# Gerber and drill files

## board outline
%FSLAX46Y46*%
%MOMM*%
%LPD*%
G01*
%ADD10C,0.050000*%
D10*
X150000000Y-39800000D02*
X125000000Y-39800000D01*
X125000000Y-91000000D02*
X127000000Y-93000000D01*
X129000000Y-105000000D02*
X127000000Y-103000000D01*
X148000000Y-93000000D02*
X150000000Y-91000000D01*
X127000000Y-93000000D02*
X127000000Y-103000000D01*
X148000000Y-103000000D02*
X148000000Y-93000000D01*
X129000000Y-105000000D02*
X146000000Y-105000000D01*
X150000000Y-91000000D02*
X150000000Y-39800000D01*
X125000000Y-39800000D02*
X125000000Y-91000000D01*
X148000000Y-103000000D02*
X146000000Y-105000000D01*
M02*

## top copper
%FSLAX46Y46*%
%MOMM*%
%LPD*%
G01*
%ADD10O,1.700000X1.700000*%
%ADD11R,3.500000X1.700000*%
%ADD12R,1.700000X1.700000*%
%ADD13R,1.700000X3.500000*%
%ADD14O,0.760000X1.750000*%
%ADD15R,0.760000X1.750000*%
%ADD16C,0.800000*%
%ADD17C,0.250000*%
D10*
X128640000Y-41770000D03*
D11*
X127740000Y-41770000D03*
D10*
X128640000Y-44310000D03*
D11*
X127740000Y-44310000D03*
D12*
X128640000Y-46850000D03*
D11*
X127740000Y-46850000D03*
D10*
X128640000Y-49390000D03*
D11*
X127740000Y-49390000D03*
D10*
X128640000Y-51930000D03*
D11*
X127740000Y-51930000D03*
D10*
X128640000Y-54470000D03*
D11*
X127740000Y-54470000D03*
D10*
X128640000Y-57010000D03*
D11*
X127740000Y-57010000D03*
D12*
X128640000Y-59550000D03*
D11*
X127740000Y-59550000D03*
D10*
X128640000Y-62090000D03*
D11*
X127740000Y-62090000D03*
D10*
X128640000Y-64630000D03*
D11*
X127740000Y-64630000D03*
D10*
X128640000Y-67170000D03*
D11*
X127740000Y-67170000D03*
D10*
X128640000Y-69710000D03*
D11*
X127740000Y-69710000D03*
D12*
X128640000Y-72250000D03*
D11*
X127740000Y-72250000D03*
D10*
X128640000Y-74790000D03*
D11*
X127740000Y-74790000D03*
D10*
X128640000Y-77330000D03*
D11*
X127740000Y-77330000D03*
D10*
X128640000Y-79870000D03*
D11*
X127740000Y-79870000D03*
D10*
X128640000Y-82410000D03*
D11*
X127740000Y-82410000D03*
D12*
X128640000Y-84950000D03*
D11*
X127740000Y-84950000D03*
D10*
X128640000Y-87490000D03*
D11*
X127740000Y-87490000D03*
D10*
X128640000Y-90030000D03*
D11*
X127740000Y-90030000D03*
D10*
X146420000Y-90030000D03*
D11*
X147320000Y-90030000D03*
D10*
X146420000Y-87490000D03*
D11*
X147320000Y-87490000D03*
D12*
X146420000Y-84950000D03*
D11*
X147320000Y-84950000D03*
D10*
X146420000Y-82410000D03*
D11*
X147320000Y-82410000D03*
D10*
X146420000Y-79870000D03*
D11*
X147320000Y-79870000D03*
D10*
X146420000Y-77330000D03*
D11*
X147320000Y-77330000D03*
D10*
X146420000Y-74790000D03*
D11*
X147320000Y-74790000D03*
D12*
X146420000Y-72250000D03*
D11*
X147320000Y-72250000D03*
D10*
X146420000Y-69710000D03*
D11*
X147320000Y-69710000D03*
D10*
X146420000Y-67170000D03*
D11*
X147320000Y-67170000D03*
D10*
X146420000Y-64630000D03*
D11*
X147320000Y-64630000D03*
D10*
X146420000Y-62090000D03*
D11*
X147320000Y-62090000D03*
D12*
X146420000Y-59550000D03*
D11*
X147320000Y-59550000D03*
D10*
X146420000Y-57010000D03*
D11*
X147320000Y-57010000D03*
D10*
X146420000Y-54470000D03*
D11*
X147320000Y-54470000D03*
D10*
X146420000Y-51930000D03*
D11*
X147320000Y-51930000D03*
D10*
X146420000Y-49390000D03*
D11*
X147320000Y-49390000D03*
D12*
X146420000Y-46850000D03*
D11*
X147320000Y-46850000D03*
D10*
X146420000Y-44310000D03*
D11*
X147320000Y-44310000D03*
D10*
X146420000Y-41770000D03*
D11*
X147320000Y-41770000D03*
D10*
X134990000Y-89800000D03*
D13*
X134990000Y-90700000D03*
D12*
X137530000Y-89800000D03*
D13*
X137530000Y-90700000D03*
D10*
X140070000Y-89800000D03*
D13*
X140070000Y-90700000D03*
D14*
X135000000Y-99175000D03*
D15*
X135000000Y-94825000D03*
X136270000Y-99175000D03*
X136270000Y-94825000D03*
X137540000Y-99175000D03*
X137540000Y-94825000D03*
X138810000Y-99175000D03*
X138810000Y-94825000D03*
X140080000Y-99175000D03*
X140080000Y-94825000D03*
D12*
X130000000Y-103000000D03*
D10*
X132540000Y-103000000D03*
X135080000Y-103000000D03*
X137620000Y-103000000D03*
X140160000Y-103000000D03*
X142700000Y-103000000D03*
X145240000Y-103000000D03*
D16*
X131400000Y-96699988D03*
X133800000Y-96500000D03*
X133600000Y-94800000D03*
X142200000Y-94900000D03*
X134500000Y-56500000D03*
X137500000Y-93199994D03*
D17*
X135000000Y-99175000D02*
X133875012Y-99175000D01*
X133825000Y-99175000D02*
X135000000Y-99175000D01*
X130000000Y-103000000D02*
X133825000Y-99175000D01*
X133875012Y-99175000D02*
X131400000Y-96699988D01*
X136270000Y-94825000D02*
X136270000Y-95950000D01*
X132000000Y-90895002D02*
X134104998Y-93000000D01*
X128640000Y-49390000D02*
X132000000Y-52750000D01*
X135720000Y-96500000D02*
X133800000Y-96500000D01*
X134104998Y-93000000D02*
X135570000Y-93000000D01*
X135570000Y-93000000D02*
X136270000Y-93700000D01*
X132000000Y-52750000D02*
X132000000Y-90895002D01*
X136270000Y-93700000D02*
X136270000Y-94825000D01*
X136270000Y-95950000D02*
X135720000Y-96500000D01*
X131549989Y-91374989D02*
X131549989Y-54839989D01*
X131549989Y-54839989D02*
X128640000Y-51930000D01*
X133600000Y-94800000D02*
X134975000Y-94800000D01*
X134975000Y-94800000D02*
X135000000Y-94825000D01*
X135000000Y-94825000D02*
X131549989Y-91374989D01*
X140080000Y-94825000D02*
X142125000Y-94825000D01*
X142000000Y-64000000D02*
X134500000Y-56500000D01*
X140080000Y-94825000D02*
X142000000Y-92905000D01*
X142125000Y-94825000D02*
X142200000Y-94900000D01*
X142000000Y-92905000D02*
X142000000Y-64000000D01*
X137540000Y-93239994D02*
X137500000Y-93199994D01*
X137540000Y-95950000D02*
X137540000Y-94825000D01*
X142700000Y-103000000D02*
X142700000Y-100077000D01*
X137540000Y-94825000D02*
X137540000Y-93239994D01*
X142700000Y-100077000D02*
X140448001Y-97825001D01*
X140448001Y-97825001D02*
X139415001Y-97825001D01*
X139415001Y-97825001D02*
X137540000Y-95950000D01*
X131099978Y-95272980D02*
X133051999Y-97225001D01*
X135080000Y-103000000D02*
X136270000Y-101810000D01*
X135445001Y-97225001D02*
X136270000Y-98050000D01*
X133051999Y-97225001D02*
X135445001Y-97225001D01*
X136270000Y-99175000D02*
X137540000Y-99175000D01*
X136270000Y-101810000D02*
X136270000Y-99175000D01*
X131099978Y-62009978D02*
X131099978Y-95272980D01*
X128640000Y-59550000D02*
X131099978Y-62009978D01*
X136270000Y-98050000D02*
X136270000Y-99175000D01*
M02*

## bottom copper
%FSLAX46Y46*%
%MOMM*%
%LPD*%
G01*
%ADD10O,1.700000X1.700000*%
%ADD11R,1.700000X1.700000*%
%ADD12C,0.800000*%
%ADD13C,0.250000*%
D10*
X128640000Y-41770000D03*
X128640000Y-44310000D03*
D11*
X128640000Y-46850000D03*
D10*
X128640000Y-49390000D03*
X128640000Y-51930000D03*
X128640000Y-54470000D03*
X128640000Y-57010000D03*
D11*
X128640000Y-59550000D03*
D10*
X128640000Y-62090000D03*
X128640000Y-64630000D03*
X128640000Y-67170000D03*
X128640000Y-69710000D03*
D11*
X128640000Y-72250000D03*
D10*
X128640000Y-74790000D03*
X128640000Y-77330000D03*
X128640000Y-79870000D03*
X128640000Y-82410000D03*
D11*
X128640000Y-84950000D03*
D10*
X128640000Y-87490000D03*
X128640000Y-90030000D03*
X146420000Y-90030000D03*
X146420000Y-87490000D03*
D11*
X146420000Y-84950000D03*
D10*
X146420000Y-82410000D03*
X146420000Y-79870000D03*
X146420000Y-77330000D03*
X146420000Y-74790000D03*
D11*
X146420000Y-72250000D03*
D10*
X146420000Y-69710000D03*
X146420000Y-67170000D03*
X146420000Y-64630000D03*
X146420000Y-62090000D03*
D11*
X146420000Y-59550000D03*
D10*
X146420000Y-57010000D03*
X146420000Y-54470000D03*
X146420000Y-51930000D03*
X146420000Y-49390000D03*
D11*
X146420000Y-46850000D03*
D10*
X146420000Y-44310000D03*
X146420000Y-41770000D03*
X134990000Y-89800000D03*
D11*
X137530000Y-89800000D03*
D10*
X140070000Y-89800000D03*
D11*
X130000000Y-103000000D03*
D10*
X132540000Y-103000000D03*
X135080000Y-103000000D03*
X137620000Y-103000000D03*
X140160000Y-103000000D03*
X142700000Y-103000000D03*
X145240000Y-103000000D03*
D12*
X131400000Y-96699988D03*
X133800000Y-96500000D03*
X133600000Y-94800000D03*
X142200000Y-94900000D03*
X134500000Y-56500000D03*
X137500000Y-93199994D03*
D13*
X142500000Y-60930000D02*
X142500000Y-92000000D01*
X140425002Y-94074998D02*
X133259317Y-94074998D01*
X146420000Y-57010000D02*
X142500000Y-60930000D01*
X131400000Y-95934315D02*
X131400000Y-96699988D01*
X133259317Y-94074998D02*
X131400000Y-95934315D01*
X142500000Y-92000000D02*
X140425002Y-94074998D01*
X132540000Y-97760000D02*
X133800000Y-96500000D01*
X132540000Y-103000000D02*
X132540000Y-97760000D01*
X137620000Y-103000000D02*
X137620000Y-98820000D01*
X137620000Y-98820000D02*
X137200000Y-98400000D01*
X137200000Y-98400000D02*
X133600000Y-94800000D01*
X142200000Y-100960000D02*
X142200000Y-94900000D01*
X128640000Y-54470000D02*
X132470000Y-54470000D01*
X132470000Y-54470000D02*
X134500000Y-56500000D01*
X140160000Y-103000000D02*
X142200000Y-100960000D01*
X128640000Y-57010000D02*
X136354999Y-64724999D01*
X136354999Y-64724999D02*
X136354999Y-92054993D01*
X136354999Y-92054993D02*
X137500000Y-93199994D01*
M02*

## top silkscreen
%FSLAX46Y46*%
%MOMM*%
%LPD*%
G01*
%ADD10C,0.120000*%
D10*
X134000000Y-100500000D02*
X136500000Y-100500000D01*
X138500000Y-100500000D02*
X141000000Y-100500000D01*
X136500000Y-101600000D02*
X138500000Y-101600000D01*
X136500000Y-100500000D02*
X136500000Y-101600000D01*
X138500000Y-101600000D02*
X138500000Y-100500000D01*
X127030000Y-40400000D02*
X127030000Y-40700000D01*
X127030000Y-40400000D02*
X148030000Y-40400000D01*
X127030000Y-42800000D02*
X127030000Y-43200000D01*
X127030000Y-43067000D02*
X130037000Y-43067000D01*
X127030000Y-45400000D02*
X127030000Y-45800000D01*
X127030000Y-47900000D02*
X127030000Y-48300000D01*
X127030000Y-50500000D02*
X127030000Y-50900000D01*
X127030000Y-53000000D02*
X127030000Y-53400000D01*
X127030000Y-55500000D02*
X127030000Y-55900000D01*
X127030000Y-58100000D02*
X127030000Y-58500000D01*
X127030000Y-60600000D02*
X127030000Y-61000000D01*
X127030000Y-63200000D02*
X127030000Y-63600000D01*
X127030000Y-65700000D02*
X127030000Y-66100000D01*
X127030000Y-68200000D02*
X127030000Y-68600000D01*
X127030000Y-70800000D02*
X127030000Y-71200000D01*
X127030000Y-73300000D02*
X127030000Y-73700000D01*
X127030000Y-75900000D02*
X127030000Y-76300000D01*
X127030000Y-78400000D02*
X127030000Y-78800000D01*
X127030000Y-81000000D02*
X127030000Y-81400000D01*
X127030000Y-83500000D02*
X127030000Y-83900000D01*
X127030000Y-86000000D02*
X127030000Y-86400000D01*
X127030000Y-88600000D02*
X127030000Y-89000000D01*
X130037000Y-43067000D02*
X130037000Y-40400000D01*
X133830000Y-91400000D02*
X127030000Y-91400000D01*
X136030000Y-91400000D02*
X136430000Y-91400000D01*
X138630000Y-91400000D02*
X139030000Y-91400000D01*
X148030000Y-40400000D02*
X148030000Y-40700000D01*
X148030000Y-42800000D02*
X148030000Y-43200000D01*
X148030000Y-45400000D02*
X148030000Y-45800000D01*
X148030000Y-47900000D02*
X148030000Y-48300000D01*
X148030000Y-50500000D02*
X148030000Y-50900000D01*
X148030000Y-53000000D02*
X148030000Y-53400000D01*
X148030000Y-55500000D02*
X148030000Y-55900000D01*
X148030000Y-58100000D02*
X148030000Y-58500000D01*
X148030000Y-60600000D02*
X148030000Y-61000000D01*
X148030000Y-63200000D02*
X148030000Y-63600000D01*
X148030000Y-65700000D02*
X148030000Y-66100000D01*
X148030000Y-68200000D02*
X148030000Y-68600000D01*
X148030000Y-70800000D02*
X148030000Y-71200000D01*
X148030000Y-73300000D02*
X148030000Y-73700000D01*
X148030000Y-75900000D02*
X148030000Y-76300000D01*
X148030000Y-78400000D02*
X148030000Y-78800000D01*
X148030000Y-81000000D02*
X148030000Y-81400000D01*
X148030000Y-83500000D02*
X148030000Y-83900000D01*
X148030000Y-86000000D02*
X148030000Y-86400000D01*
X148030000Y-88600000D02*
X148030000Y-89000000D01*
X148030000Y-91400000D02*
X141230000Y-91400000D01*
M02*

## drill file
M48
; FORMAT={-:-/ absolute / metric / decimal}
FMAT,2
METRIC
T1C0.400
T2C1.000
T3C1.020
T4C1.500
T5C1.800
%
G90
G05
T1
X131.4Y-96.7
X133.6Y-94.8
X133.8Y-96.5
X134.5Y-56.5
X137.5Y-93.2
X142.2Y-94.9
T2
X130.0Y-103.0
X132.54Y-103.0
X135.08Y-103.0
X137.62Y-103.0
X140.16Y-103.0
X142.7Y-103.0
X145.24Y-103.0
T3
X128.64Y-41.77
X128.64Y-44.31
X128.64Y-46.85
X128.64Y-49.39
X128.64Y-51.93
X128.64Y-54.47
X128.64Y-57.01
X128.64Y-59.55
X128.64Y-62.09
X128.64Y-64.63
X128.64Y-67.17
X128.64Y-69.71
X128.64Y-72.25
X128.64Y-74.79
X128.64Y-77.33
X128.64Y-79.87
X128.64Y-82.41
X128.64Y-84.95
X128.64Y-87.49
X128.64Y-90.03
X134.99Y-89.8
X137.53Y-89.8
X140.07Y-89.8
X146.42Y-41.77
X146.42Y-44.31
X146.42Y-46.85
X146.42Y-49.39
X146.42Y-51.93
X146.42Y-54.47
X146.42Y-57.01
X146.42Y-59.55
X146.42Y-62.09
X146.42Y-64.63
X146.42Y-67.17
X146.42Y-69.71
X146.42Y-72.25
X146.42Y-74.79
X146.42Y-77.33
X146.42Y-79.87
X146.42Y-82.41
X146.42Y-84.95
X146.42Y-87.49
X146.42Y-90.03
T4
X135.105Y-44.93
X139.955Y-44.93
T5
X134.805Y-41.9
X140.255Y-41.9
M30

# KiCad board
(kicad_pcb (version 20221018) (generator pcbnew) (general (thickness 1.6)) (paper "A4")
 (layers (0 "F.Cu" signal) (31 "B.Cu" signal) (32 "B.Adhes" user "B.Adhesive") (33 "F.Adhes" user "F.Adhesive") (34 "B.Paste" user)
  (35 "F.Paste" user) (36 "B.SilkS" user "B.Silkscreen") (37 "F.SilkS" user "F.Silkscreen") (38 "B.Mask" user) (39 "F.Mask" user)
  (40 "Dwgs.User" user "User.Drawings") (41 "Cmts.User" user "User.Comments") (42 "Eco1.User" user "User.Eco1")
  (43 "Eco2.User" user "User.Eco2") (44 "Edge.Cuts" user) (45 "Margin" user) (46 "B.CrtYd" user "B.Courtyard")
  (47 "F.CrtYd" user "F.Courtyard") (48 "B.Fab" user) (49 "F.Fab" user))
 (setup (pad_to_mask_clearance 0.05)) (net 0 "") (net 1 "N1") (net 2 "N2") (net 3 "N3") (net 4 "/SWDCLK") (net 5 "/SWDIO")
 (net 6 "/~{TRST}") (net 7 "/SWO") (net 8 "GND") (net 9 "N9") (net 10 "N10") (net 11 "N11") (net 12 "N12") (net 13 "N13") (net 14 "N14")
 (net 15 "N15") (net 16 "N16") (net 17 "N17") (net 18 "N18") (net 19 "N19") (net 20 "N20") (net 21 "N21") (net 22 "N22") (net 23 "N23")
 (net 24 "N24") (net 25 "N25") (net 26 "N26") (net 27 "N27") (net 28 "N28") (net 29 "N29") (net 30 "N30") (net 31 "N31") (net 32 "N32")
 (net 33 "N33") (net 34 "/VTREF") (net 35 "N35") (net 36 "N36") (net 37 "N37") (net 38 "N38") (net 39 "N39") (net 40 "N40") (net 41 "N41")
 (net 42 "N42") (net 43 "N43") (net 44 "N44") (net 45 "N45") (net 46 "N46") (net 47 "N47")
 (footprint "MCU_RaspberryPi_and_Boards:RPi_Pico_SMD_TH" (layer "F.Cu") (at 137.53 65.9)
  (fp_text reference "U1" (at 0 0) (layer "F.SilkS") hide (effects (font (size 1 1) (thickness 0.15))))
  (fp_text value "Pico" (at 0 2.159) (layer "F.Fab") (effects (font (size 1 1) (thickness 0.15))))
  (fp_line (start -10.5 -25.5) (end -10.5 -25.2) (stroke (width 0.12) (type solid)) (layer "F.SilkS"))
  (fp_line (start -10.5 -25.5) (end 10.5 -25.5) (stroke (width 0.12) (type solid)) (layer "F.SilkS"))
  (fp_line (start -10.5 -23.1) (end -10.5 -22.7) (stroke (width 0.12) (type solid)) (layer "F.SilkS"))
  (fp_line (start -10.5 -22.833) (end -7.493 -22.833) (stroke (width 0.12) (type solid)) (layer "F.SilkS"))
  (fp_line (start -10.5 -20.5) (end -10.5 -20.1) (stroke (width 0.12) (type solid)) (layer "F.SilkS"))
  (fp_line (start -10.5 -18) (end -10.5 -17.6) (stroke (width 0.12) (type solid)) (layer "F.SilkS"))
  (fp_line (start -10.5 -15.4) (end -10.5 -15) (stroke (width 0.12) (type solid)) (layer "F.SilkS"))
  (fp_line (start -10.5 -12.9) (end -10.5 -12.5) (stroke (width 0.12) (type solid)) (layer "F.SilkS"))
  (fp_line (start -10.5 -10.4) (end -10.5 -10) (stroke (width 0.12) (type solid)) (layer "F.SilkS"))
  (fp_line (start -10.5 -7.8) (end -10.5 -7.4) (stroke (width 0.12) (type solid)) (layer "F.SilkS"))
  (fp_line (start -10.5 -5.3) (end -10.5 -4.9) (stroke (width 0.12) (type solid)) (layer "F.SilkS"))
  (fp_line (start -10.5 -2.7) (end -10.5 -2.3) (stroke (width 0.12) (type solid)) (layer "F.SilkS"))
  (fp_line (start -10.5 -0.2) (end -10.5 0.2) (stroke (width 0.12) (type solid)) (layer "F.SilkS"))
  (fp_line (start -10.5 2.3) (end -10.5 2.7) (stroke (width 0.12) (type solid)) (layer "F.SilkS"))
  (fp_line (start -10.5 4.9) (end -10.5 5.3) (stroke (width 0.12) (type solid)) (layer "F.SilkS"))
  (fp_line (start -10.5 7.4) (end -10.5 7.8) (stroke (width 0.12) (type solid)) (layer "F.SilkS"))
  (fp_line (start -10.5 10) (end -10.5 10.4) (stroke (width 0.12) (type solid)) (layer "F.SilkS"))
  (fp_line (start -10.5 12.5) (end -10.5 12.9) (stroke (width 0.12) (type solid)) (layer "F.SilkS"))
  (fp_line (start -10.5 15.1) (end -10.5 15.5) (stroke (width 0.12) (type solid)) (layer "F.SilkS"))
  (fp_line (start -10.5 17.6) (end -10.5 18) (stroke (width 0.12) (type solid)) (layer "F.SilkS"))
  (fp_line (start -10.5 20.1) (end -10.5 20.5) (stroke (width 0.12) (type solid)) (layer "F.SilkS"))
  (fp_line (start -10.5 22.7) (end -10.5 23.1) (stroke (width 0.12) (type solid)) (layer "F.SilkS"))
  (fp_line (start -7.493 -22.833) (end -7.493 -25.5) (stroke (width 0.12) (type solid)) (layer "F.SilkS"))
  (fp_line (start -3.7 25.5) (end -10.5 25.5) (stroke (width 0.12) (type solid)) (layer "F.SilkS"))
  (fp_line (start -1.5 25.5) (end -1.1 25.5) (stroke (width 0.12) (type solid)) (layer "F.SilkS"))
  (fp_line (start 1.1 25.5) (end 1.5 25.5) (stroke (width 0.12) (type solid)) (layer "F.SilkS"))
  (fp_line (start 10.5 -25.5) (end 10.5 -25.2) (stroke (width 0.12) (type solid)) (layer "F.SilkS"))
  (fp_line (start 10.5 -23.1) (end 10.5 -22.7) (stroke (width 0.12) (type solid)) (layer "F.SilkS"))
  (fp_line (start 10.5 -20.5) (end 10.5 -20.1) (stroke (width 0.12) (type solid)) (layer "F.SilkS"))
  (fp_line (start 10.5 -18) (end 10.5 -17.6) (stroke (width 0.12) (type solid)) (layer "F.SilkS"))
  (fp_line (start 10.5 -15.4) (end 10.5 -15) (stroke (width 0.12) (type solid)) (layer "F.SilkS"))
  (fp_line (start 10.5 -12.9) (end 10.5 -12.5) (stroke (width 0.12) (type solid)) (layer "F.SilkS"))
  (fp_line (start 10.5 -10.4) (end 10.5 -10) (stroke (width 0.12) (type solid)) (layer "F.SilkS"))
  (fp_line (start 10.5 -7.8) (end 10.5 -7.4) (stroke (width 0.12) (type solid)) (layer "F.SilkS"))
  (fp_line (start 10.5 -5.3) (end 10.5 -4.9) (stroke (width 0.12) (type solid)) (layer "F.SilkS"))
  (fp_line (start 10.5 -2.7) (end 10.5 -2.3) (stroke (width 0.12) (type solid)) (layer "F.SilkS"))
  (fp_line (start 10.5 -0.2) (end 10.5 0.2) (stroke (width 0.12) (type solid)) (layer "F.SilkS"))
  (fp_line (start 10.5 2.3) (end 10.5 2.7) (stroke (width 0.12) (type solid)) (layer "F.SilkS"))
  (fp_line (start 10.5 4.9) (end 10.5 5.3) (stroke (width 0.12) (type solid)) (layer "F.SilkS"))
  (fp_line (start 10.5 7.4) (end 10.5 7.8) (stroke (width 0.12) (type solid)) (layer "F.SilkS"))
  (fp_line (start 10.5 10) (end 10.5 10.4) (stroke (width 0.12) (type solid)) (layer "F.SilkS"))
  (fp_line (start 10.5 12.5) (end 10.5 12.9) (stroke (width 0.12) (type solid)) (layer "F.SilkS"))
  (fp_line (start 10.5 15.1) (end 10.5 15.5) (stroke (width 0.12) (type solid)) (layer "F.SilkS"))
  (fp_line (start 10.5 17.6) (end 10.5 18) (stroke (width 0.12) (type solid)) (layer "F.SilkS"))
  (fp_line (start 10.5 20.1) (end 10.5 20.5) (stroke (width 0.12) (type solid)) (layer "F.SilkS"))
  (fp_line (start 10.5 22.7) (end 10.5 23.1) (stroke (width 0.12) (type solid)) (layer "F.SilkS"))
  (fp_line (start 10.5 25.5) (end 3.7 25.5) (stroke (width 0.12) (type solid)) (layer "F.SilkS"))
  (pad "" np_thru_hole oval (at -2.725 -24) (size 1.8 1.8) (drill 1.8) (layers "*.Cu" "*.Mask"))
  (pad "" np_thru_hole oval (at -2.425 -20.97) (size 1.5 1.5) (drill 1.5) (layers "*.Cu" "*.Mask"))
  (pad "" np_thru_hole oval (at 2.425 -20.97) (size 1.5 1.5) (drill 1.5) (layers "*.Cu" "*.Mask"))
  (pad "" np_thru_hole oval (at 2.725 -24) (size 1.8 1.8) (drill 1.8) (layers "*.Cu" "*.Mask"))
  (pad "1" thru_hole oval (at -8.89 -24.13) (size 1.7 1.7) (drill 1.02) (layers "*.Cu" "*.Mask") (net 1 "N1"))
  (pad "1" smd rect (at -8.89 -24.13) (size 3.5 1.7) (drill (offset -0.9 0)) (layers "F.Cu" "F.Mask") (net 1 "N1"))
  (pad "2" thru_hole oval (at -8.89 -21.59) (size 1.7 1.7) (drill 1.02) (layers "*.Cu" "*.Mask") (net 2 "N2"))
  (pad "2" smd rect (at -8.89 -21.59) (size 3.5 1.7) (drill (offset -0.9 0)) (layers "F.Cu" "F.Mask") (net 2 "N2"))
  (pad "3" thru_hole rect (at -8.89 -19.05) (size 1.7 1.7) (drill 1.02) (layers "*.Cu" "*.Mask") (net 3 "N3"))
  (pad "3" smd rect (at -8.89 -19.05) (size 3.5 1.7) (drill (offset -0.9 0)) (layers "F.Cu" "F.Mask") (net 3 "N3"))
  (pad "4" thru_hole oval (at -8.89 -16.51) (size 1.7 1.7) (drill 1.02) (layers "*.Cu" "*.Mask") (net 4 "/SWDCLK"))
  (pad "4" smd rect (at -8.89 -16.51) (size 3.5 1.7) (drill (offset -0.9 0)) (layers "F.Cu" "F.Mask") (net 4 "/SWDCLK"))
  (pad "5" thru_hole oval (at -8.89 -13.97) (size 1.7 1.7) (drill 1.02) (layers "*.Cu" "*.Mask") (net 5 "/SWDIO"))
  (pad "5" smd rect (at -8.89 -13.97) (size 3.5 1.7) (drill (offset -0.9 0)) (layers "F.Cu" "F.Mask") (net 5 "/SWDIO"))
  (pad "6" thru_hole oval (at -8.89 -11.43) (size 1.7 1.7) (drill 1.02) (layers "*.Cu" "*.Mask") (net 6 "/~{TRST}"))
  (pad "6" smd rect (at -8.89 -11.43) (size 3.5 1.7) (drill (offset -0.9 0)) (layers "F.Cu" "F.Mask") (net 6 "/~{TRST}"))
  (pad "7" thru_hole oval (at -8.89 -8.89) (size 1.7 1.7) (drill 1.02) (layers "*.Cu" "*.Mask") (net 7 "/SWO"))
  (pad "7" smd rect (at -8.89 -8.89) (size 3.5 1.7) (drill (offset -0.9 0)) (layers "F.Cu" "F.Mask") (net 7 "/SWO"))
  (pad "8" thru_hole rect (at -8.89 -6.35) (size 1.7 1.7) (drill 1.02) (layers "*.Cu" "*.Mask") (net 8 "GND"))
  (pad "8" smd rect (at -8.89 -6.35) (size 3.5 1.7) (drill (offset -0.9 0)) (layers "F.Cu" "F.Mask") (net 8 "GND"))
  (pad "9" thru_hole oval (at -8.89 -3.81) (size 1.7 1.7) (drill 1.02) (layers "*.Cu" "*.Mask") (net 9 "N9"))
  (pad "9" smd rect (at -8.89 -3.81) (size 3.5 1.7) (drill (offset -0.9 0)) (layers "F.Cu" "F.Mask") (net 9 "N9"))
  (pad "10" thru_hole oval (at -8.89 -1.27) (size 1.7 1.7) (drill 1.02) (layers "*.Cu" "*.Mask") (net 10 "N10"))
  (pad "10" smd rect (at -8.89 -1.27) (size 3.5 1.7) (drill (offset -0.9 0)) (layers "F.Cu" "F.Mask") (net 10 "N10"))
  (pad "11" thru_hole oval (at -8.89 1.27) (size 1.7 1.7) (drill 1.02) (layers "*.Cu" "*.Mask") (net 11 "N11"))
  (pad "11" smd rect (at -8.89 1.27) (size 3.5 1.7) (drill (offset -0.9 0)) (layers "F.Cu" "F.Mask") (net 11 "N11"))
  (pad "12" thru_hole oval (at -8.89 3.81) (size 1.7 1.7) (drill 1.02) (layers "*.Cu" "*.Mask") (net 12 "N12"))
  (pad "12" smd rect (at -8.89 3.81) (size 3.5 1.7) (drill (offset -0.9 0)) (layers "F.Cu" "F.Mask") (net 12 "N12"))
  (pad "13" thru_hole rect (at -8.89 6.35) (size 1.7 1.7) (drill 1.02) (layers "*.Cu" "*.Mask") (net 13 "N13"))
  (pad "13" smd rect (at -8.89 6.35) (size 3.5 1.7) (drill (offset -0.9 0)) (layers "F.Cu" "F.Mask") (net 13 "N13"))
  (pad "14" thru_hole oval (at -8.89 8.89) (size 1.7 1.7) (drill 1.02) (layers "*.Cu" "*.Mask") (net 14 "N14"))
  (pad "14" smd rect (at -8.89 8.89) (size 3.5 1.7) (drill (offset -0.9 0)) (layers "F.Cu" "F.Mask") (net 14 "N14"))
  (pad "15" thru_hole oval (at -8.89 11.43) (size 1.7 1.7) (drill 1.02) (layers "*.Cu" "*.Mask") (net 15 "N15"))
  (pad "15" smd rect (at -8.89 11.43) (size 3.5 1.7) (drill (offset -0.9 0)) (layers "F.Cu" "F.Mask") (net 15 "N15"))
  (pad "16" thru_hole oval (at -8.89 13.97) (size 1.7 1.7) (drill 1.02) (layers "*.Cu" "*.Mask") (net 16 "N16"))
  (pad "16" smd rect (at -8.89 13.97) (size 3.5 1.7) (drill (offset -0.9 0)) (layers "F.Cu" "F.Mask") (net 16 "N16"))
  (pad "17" thru_hole oval (at -8.89 16.51) (size 1.7 1.7) (drill 1.02) (layers "*.Cu" "*.Mask") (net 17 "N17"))
  (pad "17" smd rect (at -8.89 16.51) (size 3.5 1.7) (drill (offset -0.9 0)) (layers "F.Cu" "F.Mask") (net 17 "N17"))
  (pad "18" thru_hole rect (at -8.89 19.05) (size 1.7 1.7) (drill 1.02) (layers "*.Cu" "*.Mask") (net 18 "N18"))
  (pad "18" smd rect (at -8.89 19.05) (size 3.5 1.7) (drill (offset -0.9 0)) (layers "F.Cu" "F.Mask") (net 18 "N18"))
  (pad "19" thru_hole oval (at -8.89 21.59) (size 1.7 1.7) (drill 1.02) (layers "*.Cu" "*.Mask") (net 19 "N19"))
  (pad "19" smd rect (at -8.89 21.59) (size 3.5 1.7) (drill (offset -0.9 0)) (layers "F.Cu" "F.Mask") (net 19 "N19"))
  (pad "20" thru_hole oval (at -8.89 24.13) (size 1.7 1.7) (drill 1.02) (layers "*.Cu" "*.Mask") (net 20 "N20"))
  (pad "20" smd rect (at -8.89 24.13) (size 3.5 1.7) (drill (offset -0.9 0)) (layers "F.Cu" "F.Mask") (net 20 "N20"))
  (pad "21" thru_hole oval (at 8.89 24.13) (size 1.7 1.7) (drill 1.02) (layers "*.Cu" "*.Mask") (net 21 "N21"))
  (pad "21" smd rect (at 8.89 24.13) (size 3.5 1.7) (drill (offset 0.9 0)) (layers "F.Cu" "F.Mask") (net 21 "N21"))
  (pad "22" thru_hole oval (at 8.89 21.59) (size 1.7 1.7) (drill 1.02) (layers "*.Cu" "*.Mask") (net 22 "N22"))
  (pad "22" smd rect (at 8.89 21.59) (size 3.5 1.7) (drill (offset 0.9 0)) (layers "F.Cu" "F.Mask") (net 22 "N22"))
  (pad "23" thru_hole rect (at 8.89 19.05) (size 1.7 1.7) (drill 1.02) (layers "*.Cu" "*.Mask") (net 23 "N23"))
  (pad "23" smd rect (at 8.89 19.05) (size 3.5 1.7) (drill (offset 0.9 0)) (layers "F.Cu" "F.Mask") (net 23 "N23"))
  (pad "24" thru_hole oval (at 8.89 16.51) (size 1.7 1.7) (drill 1.02) (layers "*.Cu" "*.Mask") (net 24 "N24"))
  (pad "24" smd rect (at 8.89 16.51) (size 3.5 1.7) (drill (offset 0.9 0)) (layers "F.Cu" "F.Mask") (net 24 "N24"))
  (pad "25" thru_hole oval (at 8.89 13.97) (size 1.7 1.7) (drill 1.02) (layers "*.Cu" "*.Mask") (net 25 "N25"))
  (pad "25" smd rect (at 8.89 13.97) (size 3.5 1.7) (drill (offset 0.9 0)) (layers "F.Cu" "F.Mask") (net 25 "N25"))
  (pad "26" thru_hole oval (at 8.89 11.43) (size 1.7 1.7) (drill 1.02) (layers "*.Cu" "*.Mask") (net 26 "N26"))
  (pad "26" smd rect (at 8.89 11.43) (size 3.5 1.7) (drill (offset 0.9 0)) (layers "F.Cu" "F.Mask") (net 26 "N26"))
  (pad "27" thru_hole oval (at 8.89 8.89) (size 1.7 1.7) (drill 1.02) (layers "*.Cu" "*.Mask") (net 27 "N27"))
  (pad "27" smd rect (at 8.89 8.89) (size 3.5 1.7) (drill (offset 0.9 0)) (layers "F.Cu" "F.Mask") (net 27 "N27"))
  (pad "28" thru_hole rect (at 8.89 6.35) (size 1.7 1.7) (drill 1.02) (layers "*.Cu" "*.Mask") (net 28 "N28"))
  (pad "28" smd rect (at 8.89 6.35) (size 3.5 1.7) (drill (offset 0.9 0)) (layers "F.Cu" "F.Mask") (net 28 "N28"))
  (pad "29" thru_hole oval (at 8.89 3.81) (size 1.7 1.7) (drill 1.02) (layers "*.Cu" "*.Mask") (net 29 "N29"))
  (pad "29" smd rect (at 8.89 3.81) (size 3.5 1.7) (drill (offset 0.9 0)) (layers "F.Cu" "F.Mask") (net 29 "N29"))
  (pad "30" thru_hole oval (at 8.89 1.27) (size 1.7 1.7) (drill 1.02) (layers "*.Cu" "*.Mask") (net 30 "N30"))
  (pad "30" smd rect (at 8.89 1.27) (size 3.5 1.7) (drill (offset 0.9 0)) (layers "F.Cu" "F.Mask") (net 30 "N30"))
  (pad "31" thru_hole oval (at 8.89 -1.27) (size 1.7 1.7) (drill 1.02) (layers "*.Cu" "*.Mask") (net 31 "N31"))
  (pad "31" smd rect (at 8.89 -1.27) (size 3.5 1.7) (drill (offset 0.9 0)) (layers "F.Cu" "F.Mask") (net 31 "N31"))
  (pad "32" thru_hole oval (at 8.89 -3.81) (size 1.7 1.7) (drill 1.02) (layers "*.Cu" "*.Mask") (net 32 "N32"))
  (pad "32" smd rect (at 8.89 -3.81) (size 3.5 1.7) (drill (offset 0.9 0)) (layers "F.Cu" "F.Mask") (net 32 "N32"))
  (pad "33" thru_hole rect (at 8.89 -6.35) (size 1.7 1.7) (drill 1.02) (layers "*.Cu" "*.Mask") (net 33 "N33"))
  (pad "33" smd rect (at 8.89 -6.35) (size 3.5 1.7) (drill (offset 0.9 0)) (layers "F.Cu" "F.Mask") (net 33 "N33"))
  (pad "34" thru_hole oval (at 8.89 -8.89) (size 1.7 1.7) (drill 1.02) (layers "*.Cu" "*.Mask") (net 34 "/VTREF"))
  (pad "34" smd rect (at 8.89 -8.89) (size 3.5 1.7) (drill (offset 0.9 0)) (layers "F.Cu" "F.Mask") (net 34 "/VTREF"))
  (pad "35" thru_hole oval (at 8.89 -11.43) (size 1.7 1.7) (drill 1.02) (layers "*.Cu" "*.Mask") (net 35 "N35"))
  (pad "35" smd rect (at 8.89 -11.43) (size 3.5 1.7) (drill (offset 0.9 0)) (layers "F.Cu" "F.Mask") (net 35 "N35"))
  (pad "36" thru_hole oval (at 8.89 -13.97) (size 1.7 1.7) (drill 1.02) (layers "*.Cu" "*.Mask") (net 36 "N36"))
  (pad "36" smd rect (at 8.89 -13.97) (size 3.5 1.7) (drill (offset 0.9 0)) (layers "F.Cu" "F.Mask") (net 36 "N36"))
  (pad "37" thru_hole oval (at 8.89 -16.51) (size 1.7 1.7) (drill 1.02) (layers "*.Cu" "*.Mask") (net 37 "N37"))
  (pad "37" smd rect (at 8.89 -16.51) (size 3.5 1.7) (drill (offset 0.9 0)) (layers "F.Cu" "F.Mask") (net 37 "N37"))
  (pad "38" thru_hole rect (at 8.89 -19.05) (size 1.7 1.7) (drill 1.02) (layers "*.Cu" "*.Mask") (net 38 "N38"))
  (pad "38" smd rect (at 8.89 -19.05) (size 3.5 1.7) (drill (offset 0.9 0)) (layers "F.Cu" "F.Mask") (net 38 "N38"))
  (pad "39" thru_hole oval (at 8.89 -21.59) (size 1.7 1.7) (drill 1.02) (layers "*.Cu" "*.Mask") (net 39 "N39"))
  (pad "39" smd rect (at 8.89 -21.59) (size 3.5 1.7) (drill (offset 0.9 0)) (layers "F.Cu" "F.Mask") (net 39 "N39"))
  (pad "40" thru_hole oval (at 8.89 -24.13) (size 1.7 1.7) (drill 1.02) (layers "*.Cu" "*.Mask") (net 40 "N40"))
  (pad "40" smd rect (at 8.89 -24.13) (size 3.5 1.7) (drill (offset 0.9 0)) (layers "F.Cu" "F.Mask") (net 40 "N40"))
  (pad "41" thru_hole oval (at -2.54 23.9) (size 1.7 1.7) (drill 1.02) (layers "*.Cu" "*.Mask") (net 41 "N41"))
  (pad "41" smd rect (at -2.54 23.9 90) (size 3.5 1.7) (drill (offset -0.9 0)) (layers "F.Cu" "F.Mask") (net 41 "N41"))
  (pad "42" thru_hole rect (at 0 23.9) (size 1.7 1.7) (drill 1.02) (layers "*.Cu" "*.Mask") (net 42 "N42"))
  (pad "42" smd rect (at 0 23.9 90) (size 3.5 1.7) (drill (offset -0.9 0)) (layers "F.Cu" "F.Mask") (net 42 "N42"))
  (pad "43" thru_hole oval (at 2.54 23.9) (size 1.7 1.7) (drill 1.02) (layers "*.Cu" "*.Mask") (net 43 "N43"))
  (pad "43" smd rect (at 2.54 23.9 90) (size 3.5 1.7) (drill (offset -0.9 0)) (layers "F.Cu" "F.Mask") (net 43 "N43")))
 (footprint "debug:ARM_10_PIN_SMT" (layer "F.Cu") (at 137.5 97)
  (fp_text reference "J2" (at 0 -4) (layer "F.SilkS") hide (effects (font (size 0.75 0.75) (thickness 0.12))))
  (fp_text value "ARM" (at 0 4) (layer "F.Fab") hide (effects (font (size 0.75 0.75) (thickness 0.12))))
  (pad "1" smd oval (at -2.5 2.175) (size 0.76 1.75) (layers "F.Cu" "F.Paste" "F.Mask") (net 34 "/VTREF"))
  (pad "2" smd rect (at -2.5 -2.175) (size 0.76 1.75) (layers "F.Cu" "F.Paste" "F.Mask") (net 5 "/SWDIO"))
  (pad "3" smd rect (at -1.23 2.175) (size 0.76 1.75) (layers "F.Cu" "F.Paste" "F.Mask") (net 8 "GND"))
  (pad "4" smd rect (at -1.23 -2.175) (size 0.76 1.75) (layers "F.Cu" "F.Paste" "F.Mask") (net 4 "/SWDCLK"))
  (pad "5" smd rect (at 0.04 2.175) (size 0.76 1.75) (layers "F.Cu" "F.Paste" "F.Mask") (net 8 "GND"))
  (pad "6" smd rect (at 0.04 -2.175) (size 0.76 1.75) (layers "F.Cu" "F.Paste" "F.Mask") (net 7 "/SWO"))
  (pad "7" smd rect (at 1.31 2.175) (size 0.76 1.75) (layers "F.Cu" "F.Paste" "F.Mask") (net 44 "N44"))
  (pad "8" smd rect (at 1.31 -2.175) (size 0.76 1.75) (layers "F.Cu" "F.Paste" "F.Mask") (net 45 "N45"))
  (pad "9" smd rect (at 2.58 2.175) (size 0.76 1.75) (layers "F.Cu" "F.Paste" "F.Mask") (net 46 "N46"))
  (pad "10" smd rect (at 2.58 -2.175) (size 0.76 1.75) (layers "F.Cu" "F.Paste" "F.Mask") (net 6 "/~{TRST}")))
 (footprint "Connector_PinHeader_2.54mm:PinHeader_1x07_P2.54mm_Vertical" (layer "B.Cu") (at 130 103 -90)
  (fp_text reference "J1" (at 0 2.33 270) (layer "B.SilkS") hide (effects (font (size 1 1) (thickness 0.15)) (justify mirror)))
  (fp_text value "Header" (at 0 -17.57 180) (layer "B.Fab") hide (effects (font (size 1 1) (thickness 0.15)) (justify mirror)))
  (pad "1" thru_hole rect (at 0 0 270) (size 1.7 1.7) (drill 1) (layers "*.Cu" "*.Mask") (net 34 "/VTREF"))
  (pad "2" thru_hole oval (at 0 -2.54 270) (size 1.7 1.7) (drill 1) (layers "*.Cu" "*.Mask") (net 4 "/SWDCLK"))
  (pad "3" thru_hole oval (at 0 -5.08 270) (size 1.7 1.7) (drill 1) (layers "*.Cu" "*.Mask") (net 8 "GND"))
  (pad "4" thru_hole oval (at 0 -7.62 270) (size 1.7 1.7) (drill 1) (layers "*.Cu" "*.Mask") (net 5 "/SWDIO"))
  (pad "5" thru_hole oval (at 0 -10.16 270) (size 1.7 1.7) (drill 1) (layers "*.Cu" "*.Mask") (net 6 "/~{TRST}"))
  (pad "6" thru_hole oval (at 0 -12.7 270) (size 1.7 1.7) (drill 1) (layers "*.Cu" "*.Mask") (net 7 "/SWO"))
  (pad "7" thru_hole oval (at 0 -15.24 270) (size 1.7 1.7) (drill 1) (layers "*.Cu" "*.Mask") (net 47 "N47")))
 (gr_line (start 134 100.5) (end 136.5 100.5) (stroke (width 0.12) (type solid)) (layer "F.SilkS"))
 (gr_line (start 138.5 100.5) (end 141 100.5) (stroke (width 0.12) (type solid)) (layer "F.SilkS"))
 (gr_line (start 136.5 101.6) (end 138.5 101.6) (stroke (width 0.12) (type solid)) (layer "F.SilkS"))
 (gr_line (start 136.5 100.5) (end 136.5 101.6) (stroke (width 0.12) (type solid)) (layer "F.SilkS"))
 (gr_line (start 138.5 101.6) (end 138.5 100.5) (stroke (width 0.12) (type solid)) (layer "F.SilkS"))
 (gr_line (start 150 39.8) (end 125 39.8) (stroke (width 0.05) (type solid)) (layer "Edge.Cuts"))
 (gr_line (start 125 91) (end 127 93) (stroke (width 0.05) (type solid)) (layer "Edge.Cuts"))
 (gr_line (start 129 105) (end 127 103) (stroke (width 0.05) (type solid)) (layer "Edge.Cuts"))
 (gr_line (start 148 93) (end 150 91) (stroke (width 0.05) (type solid)) (layer "Edge.Cuts"))
 (gr_line (start 127 93) (end 127 103) (stroke (width 0.05) (type solid)) (layer "Edge.Cuts"))
 (gr_line (start 148 103) (end 148 93) (stroke (width 0.05) (type solid)) (layer "Edge.Cuts"))
 (gr_line (start 129 105) (end 146 105) (stroke (width 0.05) (type solid)) (layer "Edge.Cuts"))
 (gr_line (start 150 91) (end 150 39.8) (stroke (width 0.05) (type solid)) (layer "Edge.Cuts"))
 (gr_line (start 125 39.8) (end 125 91) (stroke (width 0.05) (type solid)) (layer "Edge.Cuts"))
 (gr_line (start 148 103) (end 146 105) (stroke (width 0.05) (type solid)) (layer "Edge.Cuts"))
 (segment (start 135 99.175) (end 133.875012 99.175) (width 0.25) (layer "F.Cu") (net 34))
 (segment (start 133.825 99.175) (end 135 99.175) (width 0.25) (layer "F.Cu") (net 34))
 (segment (start 130 103) (end 133.825 99.175) (width 0.25) (layer "F.Cu") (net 34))
 (segment (start 133.875012 99.175) (end 131.4 96.699988) (width 0.25) (layer "F.Cu") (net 34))
 (via (at 131.4 96.699988) (size 0.8) (drill 0.4) (layers "F.Cu" "B.Cu") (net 34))
 (segment (start 142.5 60.93) (end 142.5 92) (width 0.25) (layer "B.Cu") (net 34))
 (segment (start 140.425002 94.074998) (end 133.259317 94.074998) (width 0.25) (layer "B.Cu") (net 34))
 (segment (start 146.42 57.01) (end 142.5 60.93) (width 0.25) (layer "B.Cu") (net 34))
 (segment (start 131.4 95.934315) (end 131.4 96.699988) (width 0.25) (layer "B.Cu") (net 34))
 (segment (start 133.259317 94.074998) (end 131.4 95.934315) (width 0.25) (layer "B.Cu") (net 34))
 (segment (start 142.5 92) (end 140.425002 94.074998) (width 0.25) (layer "B.Cu") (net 34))
 (segment (start 136.27 94.825) (end 136.27 95.95) (width 0.25) (layer "F.Cu") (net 4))
 (segment (start 132 90.895002) (end 134.104998 93) (width 0.25) (layer "F.Cu") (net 4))
 (segment (start 128.64 49.39) (end 132 52.75) (width 0.25) (layer "F.Cu") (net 4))
 (segment (start 135.72 96.5) (end 133.8 96.5) (width 0.25) (layer "F.Cu") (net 4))
 (segment (start 134.104998 93) (end 135.57 93) (width 0.25) (layer "F.Cu") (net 4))
 (segment (start 135.57 93) (end 136.27 93.7) (width 0.25) (layer "F.Cu") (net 4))
 (segment (start 132 52.75) (end 132 90.895002) (width 0.25) (layer "F.Cu") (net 4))
 (segment (start 136.27 93.7) (end 136.27 94.825) (width 0.25) (layer "F.Cu") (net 4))
 (segment (start 136.27 95.95) (end 135.72 96.5) (width 0.25) (layer "F.Cu") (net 4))
 (via (at 133.8 96.5) (size 0.8) (drill 0.4) (layers "F.Cu" "B.Cu") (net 4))
 (segment (start 132.54 97.76) (end 133.8 96.5) (width 0.25) (layer "B.Cu") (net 4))
 (segment (start 132.54 103) (end 132.54 97.76) (width 0.25) (layer "B.Cu") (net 4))
 (segment (start 131.549989 91.374989) (end 131.549989 54.839989) (width 0.25) (layer "F.Cu") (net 5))
 (segment (start 131.549989 54.839989) (end 128.64 51.93) (width 0.25) (layer "F.Cu") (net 5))
 (segment (start 133.6 94.8) (end 134.975 94.8) (width 0.25) (layer "F.Cu") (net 5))
 (segment (start 134.975 94.8) (end 135 94.825) (width 0.25) (layer "F.Cu") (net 5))
 (segment (start 135 94.825) (end 131.549989 91.374989) (width 0.25) (layer "F.Cu") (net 5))
 (via (at 133.6 94.8) (size 0.8) (drill 0.4) (layers "F.Cu" "B.Cu") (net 5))
 (segment (start 137.62 103) (end 137.62 98.82) (width 0.25) (layer "B.Cu") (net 5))
 (segment (start 137.62 98.82) (end 137.2 98.4) (width 0.25) (layer "B.Cu") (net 5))
 (segment (start 137.2 98.4) (end 133.6 94.8) (width 0.25) (layer "B.Cu") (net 5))
 (segment (start 140.08 94.825) (end 142.125 94.825) (width 0.25) (layer "F.Cu") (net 6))
 (segment (start 142 64) (end 134.5 56.5) (width 0.25) (layer "F.Cu") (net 6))
 (segment (start 140.08 94.825) (end 142 92.905) (width 0.25) (layer "F.Cu") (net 6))
 (segment (start 142.125 94.825) (end 142.2 94.9) (width 0.25) (layer "F.Cu") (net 6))
 (segment (start 142 92.905) (end 142 64) (width 0.25) (layer "F.Cu") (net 6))
 (via (at 142.2 94.9) (size 0.8) (drill 0.4) (layers "F.Cu" "B.Cu") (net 6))
 (via (at 134.5 56.5) (size 0.8) (drill 0.4) (layers "F.Cu" "B.Cu") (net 6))
 (segment (start 142.2 100.96) (end 142.2 94.9) (width 0.25) (layer "B.Cu") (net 6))
 (segment (start 128.64 54.47) (end 132.47 54.47) (width 0.25) (layer "B.Cu") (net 6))
 (segment (start 132.47 54.47) (end 134.5 56.5) (width 0.25) (layer "B.Cu") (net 6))
 (segment (start 140.16 103) (end 142.2 100.96) (width 0.25) (layer "B.Cu") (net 6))
 (segment (start 137.54 93.239994) (end 137.5 93.199994) (width 0.25) (layer "F.Cu") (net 7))
 (segment (start 137.54 95.95) (end 137.54 94.825) (width 0.25) (layer "F.Cu") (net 7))
 (segment (start 142.7 103) (end 142.7 100.077) (width 0.25) (layer "F.Cu") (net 7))
 (segment (start 137.54 94.825) (end 137.54 93.239994) (width 0.25) (layer "F.Cu") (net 7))
 (segment (start 142.7 100.077) (end 140.448001 97.825001) (width 0.25) (layer "F.Cu") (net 7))
 (segment (start 140.448001 97.825001) (end 139.415001 97.825001) (width 0.25) (layer "F.Cu") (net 7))
 (segment (start 139.415001 97.825001) (end 137.54 95.95) (width 0.25) (layer "F.Cu") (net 7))
 (via (at 137.5 93.199994) (size 0.8) (drill 0.4) (layers "F.Cu" "B.Cu") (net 7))
 (segment (start 128.64 57.01) (end 136.354999 64.724999) (width 0.25) (layer "B.Cu") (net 7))
 (segment (start 136.354999 64.724999) (end 136.354999 92.054993) (width 0.25) (layer "B.Cu") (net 7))
 (segment (start 136.354999 92.054993) (end 137.5 93.199994) (width 0.25) (layer "B.Cu") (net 7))
 (segment (start 131.099978 95.27298) (end 133.051999 97.225001) (width 0.25) (layer "F.Cu") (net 8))
 (segment (start 135.08 103) (end 136.27 101.81) (width 0.25) (layer "F.Cu") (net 8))
 (segment (start 135.445001 97.225001) (end 136.27 98.05) (width 0.25) (layer "F.Cu") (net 8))
 (segment (start 133.051999 97.225001) (end 135.445001 97.225001) (width 0.25) (layer "F.Cu") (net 8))
 (segment (start 136.27 99.175) (end 137.54 99.175) (width 0.25) (layer "F.Cu") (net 8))
 (segment (start 136.27 101.81) (end 136.27 99.175) (width 0.25) (layer "F.Cu") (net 8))
 (segment (start 131.099978 62.009978) (end 131.099978 95.27298) (width 0.25) (layer "F.Cu") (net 8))
 (segment (start 128.64 59.55) (end 131.099978 62.009978) (width 0.25) (layer "F.Cu") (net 8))
 (segment (start 136.27 98.05) (end 136.27 99.175) (width 0.25) (layer "F.Cu") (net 8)))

